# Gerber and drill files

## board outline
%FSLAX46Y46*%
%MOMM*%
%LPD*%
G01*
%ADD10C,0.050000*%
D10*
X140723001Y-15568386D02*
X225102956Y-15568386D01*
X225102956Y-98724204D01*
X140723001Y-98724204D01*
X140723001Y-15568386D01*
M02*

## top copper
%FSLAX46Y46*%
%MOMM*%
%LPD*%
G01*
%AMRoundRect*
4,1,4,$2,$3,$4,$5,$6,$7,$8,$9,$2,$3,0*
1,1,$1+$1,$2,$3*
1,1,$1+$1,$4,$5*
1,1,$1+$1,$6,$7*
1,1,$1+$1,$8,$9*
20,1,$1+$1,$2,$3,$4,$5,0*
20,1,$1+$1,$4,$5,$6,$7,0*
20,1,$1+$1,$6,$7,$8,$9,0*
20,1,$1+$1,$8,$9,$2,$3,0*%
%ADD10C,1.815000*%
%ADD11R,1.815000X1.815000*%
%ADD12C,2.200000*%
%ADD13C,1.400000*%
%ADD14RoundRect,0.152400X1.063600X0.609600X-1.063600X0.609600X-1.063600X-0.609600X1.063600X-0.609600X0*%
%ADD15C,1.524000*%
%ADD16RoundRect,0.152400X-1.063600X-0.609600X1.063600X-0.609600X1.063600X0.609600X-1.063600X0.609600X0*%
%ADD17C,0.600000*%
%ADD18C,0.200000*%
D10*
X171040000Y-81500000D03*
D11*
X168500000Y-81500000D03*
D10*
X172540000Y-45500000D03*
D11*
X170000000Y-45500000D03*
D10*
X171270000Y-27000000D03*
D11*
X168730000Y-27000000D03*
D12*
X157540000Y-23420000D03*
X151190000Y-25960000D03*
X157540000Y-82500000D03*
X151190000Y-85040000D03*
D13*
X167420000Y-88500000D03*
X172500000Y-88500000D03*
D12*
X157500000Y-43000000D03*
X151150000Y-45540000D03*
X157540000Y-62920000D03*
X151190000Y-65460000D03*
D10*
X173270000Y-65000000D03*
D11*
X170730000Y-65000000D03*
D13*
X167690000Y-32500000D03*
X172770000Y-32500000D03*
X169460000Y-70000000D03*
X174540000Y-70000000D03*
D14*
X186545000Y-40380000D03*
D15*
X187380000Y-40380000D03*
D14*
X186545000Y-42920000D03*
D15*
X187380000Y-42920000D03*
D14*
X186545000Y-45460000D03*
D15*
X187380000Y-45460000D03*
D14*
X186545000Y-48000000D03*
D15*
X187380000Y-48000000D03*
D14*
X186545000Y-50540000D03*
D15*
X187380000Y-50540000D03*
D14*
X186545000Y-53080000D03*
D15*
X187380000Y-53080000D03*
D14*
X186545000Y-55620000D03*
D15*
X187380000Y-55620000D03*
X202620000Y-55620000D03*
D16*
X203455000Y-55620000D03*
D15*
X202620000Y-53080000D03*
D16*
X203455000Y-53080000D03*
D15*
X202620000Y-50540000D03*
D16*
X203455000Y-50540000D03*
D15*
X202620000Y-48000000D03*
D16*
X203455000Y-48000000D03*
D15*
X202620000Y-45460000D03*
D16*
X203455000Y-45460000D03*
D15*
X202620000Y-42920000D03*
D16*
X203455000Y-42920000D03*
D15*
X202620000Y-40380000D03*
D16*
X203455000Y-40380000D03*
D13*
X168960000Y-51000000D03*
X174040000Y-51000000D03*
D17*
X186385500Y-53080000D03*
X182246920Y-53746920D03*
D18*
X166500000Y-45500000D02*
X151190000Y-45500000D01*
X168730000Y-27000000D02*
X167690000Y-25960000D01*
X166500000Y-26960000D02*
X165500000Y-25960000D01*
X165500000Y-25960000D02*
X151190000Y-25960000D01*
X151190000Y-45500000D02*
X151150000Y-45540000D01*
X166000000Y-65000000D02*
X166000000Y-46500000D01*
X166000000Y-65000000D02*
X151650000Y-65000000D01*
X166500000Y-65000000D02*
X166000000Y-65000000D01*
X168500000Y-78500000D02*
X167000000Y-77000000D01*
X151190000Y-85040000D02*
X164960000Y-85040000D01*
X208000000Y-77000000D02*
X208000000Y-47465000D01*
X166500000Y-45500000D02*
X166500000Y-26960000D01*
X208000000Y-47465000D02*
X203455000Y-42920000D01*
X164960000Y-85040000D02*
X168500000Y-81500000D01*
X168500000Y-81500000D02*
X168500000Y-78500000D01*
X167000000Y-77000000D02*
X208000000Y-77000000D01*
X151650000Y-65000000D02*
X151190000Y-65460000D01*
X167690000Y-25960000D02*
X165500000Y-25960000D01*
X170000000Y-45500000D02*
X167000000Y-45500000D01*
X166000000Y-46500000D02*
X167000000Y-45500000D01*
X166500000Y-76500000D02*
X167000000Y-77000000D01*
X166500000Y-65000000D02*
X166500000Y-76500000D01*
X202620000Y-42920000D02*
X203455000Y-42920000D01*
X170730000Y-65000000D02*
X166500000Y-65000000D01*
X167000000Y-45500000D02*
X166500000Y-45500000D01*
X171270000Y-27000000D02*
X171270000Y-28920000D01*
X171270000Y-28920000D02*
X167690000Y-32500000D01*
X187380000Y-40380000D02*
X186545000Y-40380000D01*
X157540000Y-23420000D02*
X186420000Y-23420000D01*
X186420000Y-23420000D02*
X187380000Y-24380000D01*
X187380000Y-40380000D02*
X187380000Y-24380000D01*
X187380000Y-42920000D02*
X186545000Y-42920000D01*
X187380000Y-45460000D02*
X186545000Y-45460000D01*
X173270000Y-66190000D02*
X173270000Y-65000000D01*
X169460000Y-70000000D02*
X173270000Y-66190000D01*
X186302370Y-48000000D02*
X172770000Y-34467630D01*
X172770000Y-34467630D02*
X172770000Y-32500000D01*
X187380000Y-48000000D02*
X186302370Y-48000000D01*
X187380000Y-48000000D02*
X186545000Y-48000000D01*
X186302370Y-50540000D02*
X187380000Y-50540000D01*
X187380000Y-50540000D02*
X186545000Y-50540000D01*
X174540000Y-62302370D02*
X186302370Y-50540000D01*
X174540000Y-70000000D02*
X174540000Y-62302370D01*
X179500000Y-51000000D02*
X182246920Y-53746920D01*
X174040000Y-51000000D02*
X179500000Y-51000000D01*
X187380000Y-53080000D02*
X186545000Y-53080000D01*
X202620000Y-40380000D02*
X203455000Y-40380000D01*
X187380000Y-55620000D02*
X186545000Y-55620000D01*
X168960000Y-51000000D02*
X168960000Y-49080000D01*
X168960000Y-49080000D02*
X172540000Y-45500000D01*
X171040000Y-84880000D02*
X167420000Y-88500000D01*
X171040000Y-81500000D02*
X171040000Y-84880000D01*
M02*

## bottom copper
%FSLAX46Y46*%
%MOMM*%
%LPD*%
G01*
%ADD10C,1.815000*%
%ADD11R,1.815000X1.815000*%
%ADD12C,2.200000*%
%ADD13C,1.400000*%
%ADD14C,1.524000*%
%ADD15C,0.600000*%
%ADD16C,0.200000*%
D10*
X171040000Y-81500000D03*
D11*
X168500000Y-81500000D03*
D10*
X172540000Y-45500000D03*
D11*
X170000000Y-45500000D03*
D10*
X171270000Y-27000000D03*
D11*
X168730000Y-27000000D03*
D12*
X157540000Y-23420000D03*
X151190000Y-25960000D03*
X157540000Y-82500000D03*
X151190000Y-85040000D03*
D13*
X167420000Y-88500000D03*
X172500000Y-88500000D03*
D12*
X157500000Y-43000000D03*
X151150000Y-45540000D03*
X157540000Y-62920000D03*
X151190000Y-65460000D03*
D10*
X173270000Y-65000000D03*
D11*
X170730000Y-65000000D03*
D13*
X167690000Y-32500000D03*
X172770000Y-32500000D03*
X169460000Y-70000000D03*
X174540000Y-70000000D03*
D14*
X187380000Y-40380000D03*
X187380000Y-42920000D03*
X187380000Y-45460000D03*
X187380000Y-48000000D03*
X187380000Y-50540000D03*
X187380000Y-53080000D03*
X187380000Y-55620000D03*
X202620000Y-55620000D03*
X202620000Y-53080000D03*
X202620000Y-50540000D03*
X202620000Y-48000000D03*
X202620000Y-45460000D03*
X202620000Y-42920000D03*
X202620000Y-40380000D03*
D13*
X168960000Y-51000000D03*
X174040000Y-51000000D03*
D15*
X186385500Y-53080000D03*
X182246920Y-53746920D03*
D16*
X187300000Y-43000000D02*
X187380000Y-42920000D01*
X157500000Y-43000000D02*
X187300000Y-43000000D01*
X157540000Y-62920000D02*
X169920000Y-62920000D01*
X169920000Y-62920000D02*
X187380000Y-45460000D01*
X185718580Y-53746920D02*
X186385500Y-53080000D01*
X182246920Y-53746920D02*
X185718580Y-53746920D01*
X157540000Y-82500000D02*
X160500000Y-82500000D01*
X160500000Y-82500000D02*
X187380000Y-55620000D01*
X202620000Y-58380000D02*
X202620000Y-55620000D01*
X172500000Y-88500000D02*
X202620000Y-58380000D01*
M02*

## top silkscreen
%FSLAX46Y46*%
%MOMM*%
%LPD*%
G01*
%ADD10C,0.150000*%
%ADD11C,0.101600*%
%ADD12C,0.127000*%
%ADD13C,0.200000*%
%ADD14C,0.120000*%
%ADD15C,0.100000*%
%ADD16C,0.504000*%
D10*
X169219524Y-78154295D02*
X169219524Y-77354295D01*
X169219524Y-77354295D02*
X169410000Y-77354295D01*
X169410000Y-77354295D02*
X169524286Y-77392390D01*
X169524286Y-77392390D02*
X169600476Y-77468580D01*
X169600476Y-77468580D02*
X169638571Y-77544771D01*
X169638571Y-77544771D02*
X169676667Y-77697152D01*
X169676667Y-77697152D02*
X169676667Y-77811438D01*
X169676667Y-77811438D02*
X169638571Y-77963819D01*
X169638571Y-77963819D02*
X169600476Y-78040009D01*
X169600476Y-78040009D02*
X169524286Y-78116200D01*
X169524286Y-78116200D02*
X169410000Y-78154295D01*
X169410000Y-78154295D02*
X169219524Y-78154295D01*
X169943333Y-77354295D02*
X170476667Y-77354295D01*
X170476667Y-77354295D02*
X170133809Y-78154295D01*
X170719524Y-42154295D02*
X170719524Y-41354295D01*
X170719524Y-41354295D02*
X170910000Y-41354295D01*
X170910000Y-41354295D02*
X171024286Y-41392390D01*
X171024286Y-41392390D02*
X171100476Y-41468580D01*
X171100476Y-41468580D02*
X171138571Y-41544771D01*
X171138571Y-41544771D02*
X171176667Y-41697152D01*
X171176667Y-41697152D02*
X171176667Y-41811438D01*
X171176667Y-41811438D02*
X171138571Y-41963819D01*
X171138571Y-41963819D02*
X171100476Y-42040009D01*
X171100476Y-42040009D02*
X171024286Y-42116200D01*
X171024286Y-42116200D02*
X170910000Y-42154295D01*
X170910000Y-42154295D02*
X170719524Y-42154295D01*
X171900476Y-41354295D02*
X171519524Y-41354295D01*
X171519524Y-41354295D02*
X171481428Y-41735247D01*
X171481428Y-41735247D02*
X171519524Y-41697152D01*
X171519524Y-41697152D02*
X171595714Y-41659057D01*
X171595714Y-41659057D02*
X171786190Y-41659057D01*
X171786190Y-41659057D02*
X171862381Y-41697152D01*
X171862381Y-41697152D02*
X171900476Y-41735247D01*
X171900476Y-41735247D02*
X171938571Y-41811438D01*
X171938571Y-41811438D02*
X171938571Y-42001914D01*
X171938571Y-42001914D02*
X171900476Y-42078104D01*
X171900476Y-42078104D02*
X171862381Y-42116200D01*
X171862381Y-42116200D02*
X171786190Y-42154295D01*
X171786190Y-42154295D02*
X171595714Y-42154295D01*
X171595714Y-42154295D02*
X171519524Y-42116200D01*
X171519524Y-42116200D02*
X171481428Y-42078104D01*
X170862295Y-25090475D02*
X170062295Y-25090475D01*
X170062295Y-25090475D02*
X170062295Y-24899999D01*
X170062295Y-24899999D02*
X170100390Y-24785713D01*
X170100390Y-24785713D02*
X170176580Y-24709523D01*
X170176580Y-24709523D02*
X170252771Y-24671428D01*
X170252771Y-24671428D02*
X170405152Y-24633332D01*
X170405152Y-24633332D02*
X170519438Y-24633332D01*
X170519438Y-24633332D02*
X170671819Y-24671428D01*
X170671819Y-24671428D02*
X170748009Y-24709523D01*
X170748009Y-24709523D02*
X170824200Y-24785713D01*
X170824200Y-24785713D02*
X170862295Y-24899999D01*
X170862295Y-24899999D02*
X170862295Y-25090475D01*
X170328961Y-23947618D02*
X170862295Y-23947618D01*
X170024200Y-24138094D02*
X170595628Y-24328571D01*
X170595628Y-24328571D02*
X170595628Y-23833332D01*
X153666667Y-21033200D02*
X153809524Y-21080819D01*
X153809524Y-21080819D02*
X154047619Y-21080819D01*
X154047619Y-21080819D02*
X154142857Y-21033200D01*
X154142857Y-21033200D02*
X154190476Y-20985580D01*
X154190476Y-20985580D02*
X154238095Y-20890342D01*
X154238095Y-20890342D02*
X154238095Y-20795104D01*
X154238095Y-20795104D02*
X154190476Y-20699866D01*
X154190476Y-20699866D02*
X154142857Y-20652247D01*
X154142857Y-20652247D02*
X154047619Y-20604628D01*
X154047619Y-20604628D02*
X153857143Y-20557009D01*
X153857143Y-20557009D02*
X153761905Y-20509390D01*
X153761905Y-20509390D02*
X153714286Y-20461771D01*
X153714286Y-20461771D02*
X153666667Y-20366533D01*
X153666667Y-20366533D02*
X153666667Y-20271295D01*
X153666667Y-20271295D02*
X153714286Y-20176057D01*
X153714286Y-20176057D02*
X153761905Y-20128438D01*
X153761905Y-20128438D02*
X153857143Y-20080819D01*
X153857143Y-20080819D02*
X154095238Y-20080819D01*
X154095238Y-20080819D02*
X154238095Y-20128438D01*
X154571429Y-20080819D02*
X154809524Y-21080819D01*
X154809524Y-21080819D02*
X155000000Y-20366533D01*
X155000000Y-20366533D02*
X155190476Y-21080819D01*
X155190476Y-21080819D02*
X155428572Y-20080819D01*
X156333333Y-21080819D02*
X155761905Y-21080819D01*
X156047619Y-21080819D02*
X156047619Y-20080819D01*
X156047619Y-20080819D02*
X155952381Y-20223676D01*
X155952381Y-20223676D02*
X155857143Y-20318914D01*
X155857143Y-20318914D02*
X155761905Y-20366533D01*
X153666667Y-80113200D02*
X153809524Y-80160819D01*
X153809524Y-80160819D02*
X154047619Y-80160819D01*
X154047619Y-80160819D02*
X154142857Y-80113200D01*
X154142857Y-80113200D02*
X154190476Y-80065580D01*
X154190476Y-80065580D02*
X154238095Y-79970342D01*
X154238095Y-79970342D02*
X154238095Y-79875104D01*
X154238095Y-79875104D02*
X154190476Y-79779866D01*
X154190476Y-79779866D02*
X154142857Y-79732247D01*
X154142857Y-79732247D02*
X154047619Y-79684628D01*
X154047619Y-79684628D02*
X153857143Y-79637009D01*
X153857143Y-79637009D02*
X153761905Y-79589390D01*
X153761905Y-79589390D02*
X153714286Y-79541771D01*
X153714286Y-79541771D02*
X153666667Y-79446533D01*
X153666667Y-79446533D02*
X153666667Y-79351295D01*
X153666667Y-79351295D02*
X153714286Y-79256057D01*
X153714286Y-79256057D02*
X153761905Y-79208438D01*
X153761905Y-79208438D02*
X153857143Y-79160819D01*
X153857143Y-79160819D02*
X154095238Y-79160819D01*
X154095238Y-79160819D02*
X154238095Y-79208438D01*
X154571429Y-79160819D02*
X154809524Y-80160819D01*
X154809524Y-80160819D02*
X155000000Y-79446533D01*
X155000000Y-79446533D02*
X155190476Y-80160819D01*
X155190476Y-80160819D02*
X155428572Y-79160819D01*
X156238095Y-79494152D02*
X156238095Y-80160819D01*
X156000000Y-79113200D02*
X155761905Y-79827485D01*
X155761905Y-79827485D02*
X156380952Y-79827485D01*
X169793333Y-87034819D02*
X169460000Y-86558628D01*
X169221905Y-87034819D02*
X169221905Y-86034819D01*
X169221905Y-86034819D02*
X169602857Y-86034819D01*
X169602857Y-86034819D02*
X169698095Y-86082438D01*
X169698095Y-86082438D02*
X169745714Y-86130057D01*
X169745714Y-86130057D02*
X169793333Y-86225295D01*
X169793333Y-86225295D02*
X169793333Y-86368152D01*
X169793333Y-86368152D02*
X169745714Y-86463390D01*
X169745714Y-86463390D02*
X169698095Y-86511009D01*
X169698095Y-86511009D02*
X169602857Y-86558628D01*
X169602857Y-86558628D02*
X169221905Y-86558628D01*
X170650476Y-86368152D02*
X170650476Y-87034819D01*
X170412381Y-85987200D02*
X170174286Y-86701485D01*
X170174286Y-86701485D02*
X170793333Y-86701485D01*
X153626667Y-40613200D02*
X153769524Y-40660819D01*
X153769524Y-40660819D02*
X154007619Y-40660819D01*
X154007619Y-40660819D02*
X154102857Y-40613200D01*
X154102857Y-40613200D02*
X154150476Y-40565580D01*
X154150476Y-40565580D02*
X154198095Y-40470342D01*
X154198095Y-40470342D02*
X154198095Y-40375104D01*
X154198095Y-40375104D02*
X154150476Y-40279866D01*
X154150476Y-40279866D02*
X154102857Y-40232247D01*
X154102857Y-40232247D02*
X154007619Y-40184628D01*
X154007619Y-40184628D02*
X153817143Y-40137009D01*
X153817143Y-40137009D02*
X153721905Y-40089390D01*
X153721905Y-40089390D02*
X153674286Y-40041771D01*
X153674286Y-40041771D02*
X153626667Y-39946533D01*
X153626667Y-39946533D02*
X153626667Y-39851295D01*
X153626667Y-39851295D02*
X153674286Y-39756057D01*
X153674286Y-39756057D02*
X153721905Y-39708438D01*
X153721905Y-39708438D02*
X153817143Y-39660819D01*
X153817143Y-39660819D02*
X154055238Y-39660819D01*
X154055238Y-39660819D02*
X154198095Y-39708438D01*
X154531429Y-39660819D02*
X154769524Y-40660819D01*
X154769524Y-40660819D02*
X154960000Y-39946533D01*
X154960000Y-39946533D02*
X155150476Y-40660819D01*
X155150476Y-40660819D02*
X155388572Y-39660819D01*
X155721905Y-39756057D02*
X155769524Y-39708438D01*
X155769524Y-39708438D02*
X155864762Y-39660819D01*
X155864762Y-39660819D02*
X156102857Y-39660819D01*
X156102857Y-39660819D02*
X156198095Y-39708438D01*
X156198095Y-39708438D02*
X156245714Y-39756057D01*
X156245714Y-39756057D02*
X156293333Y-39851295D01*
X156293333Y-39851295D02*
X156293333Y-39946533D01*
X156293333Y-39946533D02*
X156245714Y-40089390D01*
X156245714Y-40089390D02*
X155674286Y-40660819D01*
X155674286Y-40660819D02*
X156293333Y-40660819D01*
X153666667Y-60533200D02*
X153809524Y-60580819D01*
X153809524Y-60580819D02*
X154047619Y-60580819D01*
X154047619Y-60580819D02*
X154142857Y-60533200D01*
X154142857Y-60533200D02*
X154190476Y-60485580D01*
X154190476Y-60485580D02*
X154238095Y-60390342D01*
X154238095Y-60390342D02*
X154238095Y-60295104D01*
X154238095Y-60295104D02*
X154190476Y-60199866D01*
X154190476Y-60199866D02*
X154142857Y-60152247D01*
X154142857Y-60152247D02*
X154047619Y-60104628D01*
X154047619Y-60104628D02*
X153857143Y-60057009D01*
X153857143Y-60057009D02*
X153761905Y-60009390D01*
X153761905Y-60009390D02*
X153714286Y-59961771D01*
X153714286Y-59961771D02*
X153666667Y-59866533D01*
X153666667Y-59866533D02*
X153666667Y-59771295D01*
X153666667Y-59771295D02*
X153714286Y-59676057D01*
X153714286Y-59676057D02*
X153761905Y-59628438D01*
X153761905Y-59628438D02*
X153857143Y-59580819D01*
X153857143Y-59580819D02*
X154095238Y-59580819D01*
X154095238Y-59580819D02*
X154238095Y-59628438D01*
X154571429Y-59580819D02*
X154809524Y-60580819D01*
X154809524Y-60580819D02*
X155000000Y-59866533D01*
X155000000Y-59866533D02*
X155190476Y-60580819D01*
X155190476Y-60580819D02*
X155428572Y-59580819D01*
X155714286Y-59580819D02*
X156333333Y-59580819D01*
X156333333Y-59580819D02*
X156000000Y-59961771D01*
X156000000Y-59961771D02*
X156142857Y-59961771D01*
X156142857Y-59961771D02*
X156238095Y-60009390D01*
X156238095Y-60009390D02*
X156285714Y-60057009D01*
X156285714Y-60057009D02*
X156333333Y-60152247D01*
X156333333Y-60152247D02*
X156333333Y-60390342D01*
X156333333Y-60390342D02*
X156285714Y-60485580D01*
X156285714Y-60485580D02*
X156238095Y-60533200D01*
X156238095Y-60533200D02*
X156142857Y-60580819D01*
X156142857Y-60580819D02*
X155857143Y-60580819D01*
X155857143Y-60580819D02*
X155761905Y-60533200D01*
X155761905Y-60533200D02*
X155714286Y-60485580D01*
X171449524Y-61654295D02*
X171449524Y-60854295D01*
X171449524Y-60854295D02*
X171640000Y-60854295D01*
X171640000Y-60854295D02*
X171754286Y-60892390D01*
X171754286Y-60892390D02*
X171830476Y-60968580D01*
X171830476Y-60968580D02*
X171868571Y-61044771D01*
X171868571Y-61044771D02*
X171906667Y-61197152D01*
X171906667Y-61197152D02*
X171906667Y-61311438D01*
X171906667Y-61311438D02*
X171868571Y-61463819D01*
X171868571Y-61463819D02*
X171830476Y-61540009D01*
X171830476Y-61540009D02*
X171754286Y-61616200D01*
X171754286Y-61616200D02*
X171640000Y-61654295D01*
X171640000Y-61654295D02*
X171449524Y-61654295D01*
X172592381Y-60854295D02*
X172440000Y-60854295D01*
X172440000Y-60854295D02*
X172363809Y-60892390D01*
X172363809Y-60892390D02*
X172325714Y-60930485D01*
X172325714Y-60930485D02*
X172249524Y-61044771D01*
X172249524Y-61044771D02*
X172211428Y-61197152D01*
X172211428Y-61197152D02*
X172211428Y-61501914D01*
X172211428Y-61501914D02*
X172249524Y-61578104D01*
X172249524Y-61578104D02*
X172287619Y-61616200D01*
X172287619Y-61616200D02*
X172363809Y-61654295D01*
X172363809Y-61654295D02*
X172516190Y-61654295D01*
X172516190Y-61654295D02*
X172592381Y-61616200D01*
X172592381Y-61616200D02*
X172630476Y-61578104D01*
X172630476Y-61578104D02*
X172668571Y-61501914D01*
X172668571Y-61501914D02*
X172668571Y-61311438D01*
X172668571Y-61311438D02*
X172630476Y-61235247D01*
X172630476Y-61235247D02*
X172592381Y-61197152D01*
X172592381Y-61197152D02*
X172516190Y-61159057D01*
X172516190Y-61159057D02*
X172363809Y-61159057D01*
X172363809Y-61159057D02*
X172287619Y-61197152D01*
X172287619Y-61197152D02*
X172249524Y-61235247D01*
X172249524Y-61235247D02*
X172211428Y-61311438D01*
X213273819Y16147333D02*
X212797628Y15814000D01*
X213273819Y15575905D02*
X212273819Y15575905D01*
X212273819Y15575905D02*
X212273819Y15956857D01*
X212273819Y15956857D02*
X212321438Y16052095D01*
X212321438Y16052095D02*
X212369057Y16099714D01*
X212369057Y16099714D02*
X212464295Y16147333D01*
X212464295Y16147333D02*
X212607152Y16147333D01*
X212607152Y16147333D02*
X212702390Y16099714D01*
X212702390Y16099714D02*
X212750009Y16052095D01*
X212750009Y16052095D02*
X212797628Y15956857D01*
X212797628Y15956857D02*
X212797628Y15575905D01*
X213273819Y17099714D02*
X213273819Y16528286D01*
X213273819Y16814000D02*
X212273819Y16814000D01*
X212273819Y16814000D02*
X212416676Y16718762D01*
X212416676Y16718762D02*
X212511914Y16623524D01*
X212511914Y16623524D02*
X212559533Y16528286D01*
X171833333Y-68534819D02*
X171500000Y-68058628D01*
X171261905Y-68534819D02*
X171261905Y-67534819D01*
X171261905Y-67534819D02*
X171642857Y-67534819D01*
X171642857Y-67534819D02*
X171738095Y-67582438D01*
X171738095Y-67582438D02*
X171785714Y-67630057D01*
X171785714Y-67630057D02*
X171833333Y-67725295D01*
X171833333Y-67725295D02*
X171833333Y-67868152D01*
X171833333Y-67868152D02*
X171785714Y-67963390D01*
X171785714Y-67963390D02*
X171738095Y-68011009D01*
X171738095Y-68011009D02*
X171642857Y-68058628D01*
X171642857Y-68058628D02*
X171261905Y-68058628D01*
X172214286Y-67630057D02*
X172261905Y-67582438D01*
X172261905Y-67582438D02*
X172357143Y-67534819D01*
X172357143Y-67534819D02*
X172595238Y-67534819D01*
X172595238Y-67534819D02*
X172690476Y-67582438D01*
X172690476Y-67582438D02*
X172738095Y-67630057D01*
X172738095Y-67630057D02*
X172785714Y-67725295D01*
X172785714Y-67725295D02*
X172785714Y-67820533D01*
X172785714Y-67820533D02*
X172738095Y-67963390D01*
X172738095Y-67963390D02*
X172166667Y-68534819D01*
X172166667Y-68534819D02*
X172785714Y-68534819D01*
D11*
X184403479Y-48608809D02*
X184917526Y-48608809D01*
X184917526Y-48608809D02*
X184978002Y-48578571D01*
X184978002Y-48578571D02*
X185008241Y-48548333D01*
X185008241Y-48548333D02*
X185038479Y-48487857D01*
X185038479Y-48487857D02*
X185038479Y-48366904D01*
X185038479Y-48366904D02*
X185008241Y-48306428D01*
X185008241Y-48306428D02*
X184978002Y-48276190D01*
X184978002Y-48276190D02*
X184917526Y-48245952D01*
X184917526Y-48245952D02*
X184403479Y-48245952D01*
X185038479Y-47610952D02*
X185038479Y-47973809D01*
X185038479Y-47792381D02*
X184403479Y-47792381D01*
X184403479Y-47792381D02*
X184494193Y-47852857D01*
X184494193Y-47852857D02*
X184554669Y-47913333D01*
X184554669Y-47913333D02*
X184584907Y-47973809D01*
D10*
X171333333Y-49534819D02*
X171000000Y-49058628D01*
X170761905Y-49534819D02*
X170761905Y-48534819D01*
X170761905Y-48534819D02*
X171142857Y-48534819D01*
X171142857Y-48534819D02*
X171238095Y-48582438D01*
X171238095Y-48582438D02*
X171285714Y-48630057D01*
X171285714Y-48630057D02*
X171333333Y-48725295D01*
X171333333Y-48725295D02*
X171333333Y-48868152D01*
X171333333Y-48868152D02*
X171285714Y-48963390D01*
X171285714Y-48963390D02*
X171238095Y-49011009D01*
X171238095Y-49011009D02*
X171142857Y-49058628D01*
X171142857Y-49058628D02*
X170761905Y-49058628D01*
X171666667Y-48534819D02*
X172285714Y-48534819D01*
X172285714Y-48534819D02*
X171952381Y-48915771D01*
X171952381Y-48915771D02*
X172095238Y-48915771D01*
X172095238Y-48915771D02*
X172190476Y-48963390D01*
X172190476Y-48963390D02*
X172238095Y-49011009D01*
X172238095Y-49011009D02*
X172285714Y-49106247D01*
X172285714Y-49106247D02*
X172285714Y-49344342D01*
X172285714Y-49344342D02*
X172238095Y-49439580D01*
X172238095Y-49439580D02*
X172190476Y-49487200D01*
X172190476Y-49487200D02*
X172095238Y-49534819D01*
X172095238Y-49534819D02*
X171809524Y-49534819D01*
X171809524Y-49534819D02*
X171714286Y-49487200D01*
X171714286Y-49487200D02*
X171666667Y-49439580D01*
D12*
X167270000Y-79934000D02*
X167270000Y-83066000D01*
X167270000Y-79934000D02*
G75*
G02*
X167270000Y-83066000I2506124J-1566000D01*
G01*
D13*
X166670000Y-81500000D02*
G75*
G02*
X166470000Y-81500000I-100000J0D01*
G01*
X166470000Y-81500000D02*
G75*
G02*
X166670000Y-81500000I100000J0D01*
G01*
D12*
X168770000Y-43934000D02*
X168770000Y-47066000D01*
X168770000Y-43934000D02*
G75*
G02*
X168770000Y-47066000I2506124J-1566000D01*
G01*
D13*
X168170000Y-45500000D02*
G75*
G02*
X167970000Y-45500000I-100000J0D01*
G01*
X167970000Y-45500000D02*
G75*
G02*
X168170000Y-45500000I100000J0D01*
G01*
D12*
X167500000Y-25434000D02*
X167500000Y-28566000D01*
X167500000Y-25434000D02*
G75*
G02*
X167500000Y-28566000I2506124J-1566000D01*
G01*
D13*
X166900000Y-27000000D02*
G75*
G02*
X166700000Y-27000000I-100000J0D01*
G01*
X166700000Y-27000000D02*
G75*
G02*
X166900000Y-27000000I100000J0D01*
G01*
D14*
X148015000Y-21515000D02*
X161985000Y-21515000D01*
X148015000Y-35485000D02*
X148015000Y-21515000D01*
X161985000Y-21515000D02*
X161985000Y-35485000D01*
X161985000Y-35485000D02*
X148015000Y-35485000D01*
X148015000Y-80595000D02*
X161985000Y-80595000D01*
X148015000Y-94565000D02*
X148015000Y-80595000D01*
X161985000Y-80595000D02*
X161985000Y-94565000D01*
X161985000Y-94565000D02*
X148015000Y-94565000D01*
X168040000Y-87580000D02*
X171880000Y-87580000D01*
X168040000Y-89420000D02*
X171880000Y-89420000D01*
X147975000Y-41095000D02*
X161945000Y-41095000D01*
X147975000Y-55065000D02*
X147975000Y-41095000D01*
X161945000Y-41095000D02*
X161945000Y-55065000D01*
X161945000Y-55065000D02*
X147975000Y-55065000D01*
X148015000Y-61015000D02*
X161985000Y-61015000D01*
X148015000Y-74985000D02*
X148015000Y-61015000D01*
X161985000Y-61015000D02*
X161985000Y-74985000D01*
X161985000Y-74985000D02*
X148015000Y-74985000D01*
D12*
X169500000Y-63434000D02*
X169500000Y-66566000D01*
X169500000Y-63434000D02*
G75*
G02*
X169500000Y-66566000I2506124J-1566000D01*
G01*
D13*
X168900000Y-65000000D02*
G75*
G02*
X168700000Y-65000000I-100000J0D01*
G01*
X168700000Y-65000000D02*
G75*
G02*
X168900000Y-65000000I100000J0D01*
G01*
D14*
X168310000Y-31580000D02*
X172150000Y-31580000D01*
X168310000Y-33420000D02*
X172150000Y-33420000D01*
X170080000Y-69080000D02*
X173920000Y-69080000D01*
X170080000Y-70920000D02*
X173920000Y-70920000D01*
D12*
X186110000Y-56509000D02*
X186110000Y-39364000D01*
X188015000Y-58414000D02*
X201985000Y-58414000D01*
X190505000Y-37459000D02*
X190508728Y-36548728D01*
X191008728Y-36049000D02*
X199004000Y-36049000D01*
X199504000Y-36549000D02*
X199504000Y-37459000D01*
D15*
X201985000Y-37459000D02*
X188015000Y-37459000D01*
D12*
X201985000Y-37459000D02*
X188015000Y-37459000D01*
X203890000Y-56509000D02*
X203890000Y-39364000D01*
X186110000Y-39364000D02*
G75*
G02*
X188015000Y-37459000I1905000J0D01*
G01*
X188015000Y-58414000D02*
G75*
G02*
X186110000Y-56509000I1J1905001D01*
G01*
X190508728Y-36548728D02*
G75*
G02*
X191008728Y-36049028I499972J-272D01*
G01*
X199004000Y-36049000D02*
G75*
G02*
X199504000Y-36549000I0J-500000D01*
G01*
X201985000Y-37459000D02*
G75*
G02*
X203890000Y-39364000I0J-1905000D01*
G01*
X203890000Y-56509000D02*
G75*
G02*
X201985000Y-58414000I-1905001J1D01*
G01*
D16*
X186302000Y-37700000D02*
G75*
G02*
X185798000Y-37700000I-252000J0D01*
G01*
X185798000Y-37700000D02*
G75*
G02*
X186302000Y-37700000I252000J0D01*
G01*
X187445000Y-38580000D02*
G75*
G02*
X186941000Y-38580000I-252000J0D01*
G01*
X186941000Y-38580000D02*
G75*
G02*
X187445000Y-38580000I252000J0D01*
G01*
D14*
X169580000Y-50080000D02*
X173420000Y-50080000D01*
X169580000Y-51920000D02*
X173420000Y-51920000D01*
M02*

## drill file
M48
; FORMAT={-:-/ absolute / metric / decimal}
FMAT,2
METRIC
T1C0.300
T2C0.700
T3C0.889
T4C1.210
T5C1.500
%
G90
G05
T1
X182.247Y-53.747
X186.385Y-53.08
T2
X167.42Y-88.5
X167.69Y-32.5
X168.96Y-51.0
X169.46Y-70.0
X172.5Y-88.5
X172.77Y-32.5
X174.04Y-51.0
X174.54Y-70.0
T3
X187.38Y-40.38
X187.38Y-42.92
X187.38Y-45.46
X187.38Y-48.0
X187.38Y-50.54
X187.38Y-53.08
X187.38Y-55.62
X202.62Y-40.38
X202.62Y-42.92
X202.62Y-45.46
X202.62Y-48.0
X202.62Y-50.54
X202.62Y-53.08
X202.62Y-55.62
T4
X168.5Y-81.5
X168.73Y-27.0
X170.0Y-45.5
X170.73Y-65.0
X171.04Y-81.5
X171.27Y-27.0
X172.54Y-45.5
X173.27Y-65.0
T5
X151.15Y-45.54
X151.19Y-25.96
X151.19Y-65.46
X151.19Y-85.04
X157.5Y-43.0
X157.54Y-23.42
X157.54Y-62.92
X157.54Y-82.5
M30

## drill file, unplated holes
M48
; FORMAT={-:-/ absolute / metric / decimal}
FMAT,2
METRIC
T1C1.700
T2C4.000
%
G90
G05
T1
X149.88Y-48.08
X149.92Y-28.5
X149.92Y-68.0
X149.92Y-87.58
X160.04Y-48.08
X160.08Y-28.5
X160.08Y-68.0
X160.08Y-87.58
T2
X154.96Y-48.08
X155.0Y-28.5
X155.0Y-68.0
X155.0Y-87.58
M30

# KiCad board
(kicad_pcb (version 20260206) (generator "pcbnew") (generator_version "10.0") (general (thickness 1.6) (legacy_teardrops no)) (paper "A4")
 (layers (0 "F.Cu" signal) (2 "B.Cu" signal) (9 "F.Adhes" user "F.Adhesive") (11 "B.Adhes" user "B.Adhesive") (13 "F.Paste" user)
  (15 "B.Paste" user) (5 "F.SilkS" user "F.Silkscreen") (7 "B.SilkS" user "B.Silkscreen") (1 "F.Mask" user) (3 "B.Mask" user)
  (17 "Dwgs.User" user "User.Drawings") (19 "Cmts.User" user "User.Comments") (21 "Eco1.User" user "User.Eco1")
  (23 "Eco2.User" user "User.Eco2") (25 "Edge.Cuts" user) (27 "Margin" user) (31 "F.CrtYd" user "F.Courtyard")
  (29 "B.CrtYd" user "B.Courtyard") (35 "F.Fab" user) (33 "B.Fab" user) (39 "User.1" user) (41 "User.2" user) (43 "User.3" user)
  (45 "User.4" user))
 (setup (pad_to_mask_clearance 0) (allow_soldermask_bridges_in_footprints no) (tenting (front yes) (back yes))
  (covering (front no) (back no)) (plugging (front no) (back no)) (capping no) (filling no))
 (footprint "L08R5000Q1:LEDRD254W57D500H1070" (layer "F.Cu") (at 169.77 81.5)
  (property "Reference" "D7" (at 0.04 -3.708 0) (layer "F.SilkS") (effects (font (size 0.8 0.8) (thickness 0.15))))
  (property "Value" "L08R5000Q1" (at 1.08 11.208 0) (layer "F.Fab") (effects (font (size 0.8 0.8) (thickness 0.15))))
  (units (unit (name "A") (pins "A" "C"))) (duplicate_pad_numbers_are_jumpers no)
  (fp_line (start -2.5 -1.566) (end -2.5 1.566) (stroke (width 0.127) (type solid)) (layer "F.SilkS"))
  (fp_arc (start -2.5 -1.566) (mid 2.961291 0) (end -2.5 1.566) (stroke (width 0.127) (type solid)) (layer "F.SilkS"))
  (fp_circle (center -3.2 0) (end -3.1 0) (stroke (width 0.2) (type solid)) (fill no) (layer "F.SilkS"))
  (pad "A" thru_hole circle (at 1.27 0) (size 1.815 1.815) (drill 1.21) (layers "*.Cu" "*.Mask") (remove_unused_layers no)
   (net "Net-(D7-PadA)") (solder_mask_margin 0.102))
  (pad "C" thru_hole rect (at -1.27 0) (size 1.815 1.815) (drill 1.21) (layers "*.Cu" "*.Mask") (remove_unused_layers no) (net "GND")
   (solder_mask_margin 0.102)))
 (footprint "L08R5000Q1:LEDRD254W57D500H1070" (layer "F.Cu") (at 171.27 45.5)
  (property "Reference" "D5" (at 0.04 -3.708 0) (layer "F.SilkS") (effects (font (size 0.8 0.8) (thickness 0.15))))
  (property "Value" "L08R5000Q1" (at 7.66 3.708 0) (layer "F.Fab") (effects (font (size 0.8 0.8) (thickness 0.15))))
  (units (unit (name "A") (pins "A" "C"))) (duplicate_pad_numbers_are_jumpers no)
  (fp_line (start -2.5 -1.566) (end -2.5 1.566) (stroke (width 0.127) (type solid)) (layer "F.SilkS"))
  (fp_arc (start -2.5 -1.566) (mid 2.961291 0) (end -2.5 1.566) (stroke (width 0.127) (type solid)) (layer "F.SilkS"))
  (fp_circle (center -3.2 0) (end -3.1 0) (stroke (width 0.2) (type solid)) (fill no) (layer "F.SilkS"))
  (pad "A" thru_hole circle (at 1.27 0) (size 1.815 1.815) (drill 1.21) (layers "*.Cu" "*.Mask") (remove_unused_layers no)
   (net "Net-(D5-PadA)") (solder_mask_margin 0.102))
  (pad "C" thru_hole rect (at -1.27 0) (size 1.815 1.815) (drill 1.21) (layers "*.Cu" "*.Mask") (remove_unused_layers no) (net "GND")
   (solder_mask_margin 0.102)))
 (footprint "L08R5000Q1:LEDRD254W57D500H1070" (layer "F.Cu") (at 170 27)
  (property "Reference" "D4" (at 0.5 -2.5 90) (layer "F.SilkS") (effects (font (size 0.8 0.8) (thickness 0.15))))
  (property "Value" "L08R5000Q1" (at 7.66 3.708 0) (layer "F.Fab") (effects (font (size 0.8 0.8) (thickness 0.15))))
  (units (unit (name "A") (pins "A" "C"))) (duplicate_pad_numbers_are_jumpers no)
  (fp_line (start -2.5 -1.566) (end -2.5 1.566) (stroke (width 0.127) (type solid)) (layer "F.SilkS"))
  (fp_arc (start -2.5 -1.566) (mid 2.961291 0) (end -2.5 1.566) (stroke (width 0.127) (type solid)) (layer "F.SilkS"))
  (fp_circle (center -3.2 0) (end -3.1 0) (stroke (width 0.2) (type solid)) (fill no) (layer "F.SilkS"))
  (pad "A" thru_hole circle (at 1.27 0) (size 1.815 1.815) (drill 1.21) (layers "*.Cu" "*.Mask") (remove_unused_layers no)
   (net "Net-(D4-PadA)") (solder_mask_margin 0.102))
  (pad "C" thru_hole rect (at -1.27 0) (size 1.815 1.815) (drill 1.21) (layers "*.Cu" "*.Mask") (remove_unused_layers no) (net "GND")
   (solder_mask_margin 0.102)))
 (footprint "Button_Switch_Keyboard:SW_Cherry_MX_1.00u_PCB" (layer "F.Cu") (at 157.54 23.42)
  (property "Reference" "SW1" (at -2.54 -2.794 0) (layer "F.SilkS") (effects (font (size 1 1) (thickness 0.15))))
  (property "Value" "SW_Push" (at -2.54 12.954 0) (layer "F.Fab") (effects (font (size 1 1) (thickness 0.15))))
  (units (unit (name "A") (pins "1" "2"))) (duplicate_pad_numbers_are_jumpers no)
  (fp_line (start -9.525 -1.905) (end 4.445 -1.905) (stroke (width 0.12) (type solid)) (layer "F.SilkS"))
  (fp_line (start -9.525 12.065) (end -9.525 -1.905) (stroke (width 0.12) (type solid)) (layer "F.SilkS"))
  (fp_line (start 4.445 -1.905) (end 4.445 12.065) (stroke (width 0.12) (type solid)) (layer "F.SilkS"))
  (fp_line (start 4.445 12.065) (end -9.525 12.065) (stroke (width 0.12) (type solid)) (layer "F.SilkS"))
  (pad "" np_thru_hole circle (at -7.62 5.08) (size 1.7 1.7) (drill 1.7) (layers "*.Cu" "*.Mask"))
  (pad "" np_thru_hole circle (at -2.54 5.08) (size 4 4) (drill 4) (layers "*.Cu" "*.Mask"))
  (pad "" np_thru_hole circle (at 2.54 5.08) (size 1.7 1.7) (drill 1.7) (layers "*.Cu" "*.Mask"))
  (pad "1" thru_hole circle (at 0 0) (size 2.2 2.2) (drill 1.5) (layers "*.Cu" "*.Mask") (remove_unused_layers no) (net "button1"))
  (pad "2" thru_hole circle (at -6.35 2.54) (size 2.2 2.2) (drill 1.5) (layers "*.Cu" "*.Mask") (remove_unused_layers no) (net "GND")))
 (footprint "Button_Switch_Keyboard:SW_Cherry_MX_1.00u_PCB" (layer "F.Cu") (at 157.54 82.5)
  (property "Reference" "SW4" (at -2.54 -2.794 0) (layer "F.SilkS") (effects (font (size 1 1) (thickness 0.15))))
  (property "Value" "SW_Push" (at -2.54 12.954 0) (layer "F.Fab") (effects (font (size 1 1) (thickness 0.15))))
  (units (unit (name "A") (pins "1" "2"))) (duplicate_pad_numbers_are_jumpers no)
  (fp_line (start -9.525 -1.905) (end 4.445 -1.905) (stroke (width 0.12) (type solid)) (layer "F.SilkS"))
  (fp_line (start -9.525 12.065) (end -9.525 -1.905) (stroke (width 0.12) (type solid)) (layer "F.SilkS"))
  (fp_line (start 4.445 -1.905) (end 4.445 12.065) (stroke (width 0.12) (type solid)) (layer "F.SilkS"))
  (fp_line (start 4.445 12.065) (end -9.525 12.065) (stroke (width 0.12) (type solid)) (layer "F.SilkS"))
  (pad "" np_thru_hole circle (at -7.62 5.08) (size 1.7 1.7) (drill 1.7) (layers "*.Cu" "*.Mask"))
  (pad "" np_thru_hole circle (at -2.54 5.08) (size 4 4) (drill 4) (layers "*.Cu" "*.Mask"))
  (pad "" np_thru_hole circle (at 2.54 5.08) (size 1.7 1.7) (drill 1.7) (layers "*.Cu" "*.Mask"))
  (pad "1" thru_hole circle (at 0 0) (size 2.2 2.2) (drill 1.5) (layers "*.Cu" "*.Mask") (remove_unused_layers no) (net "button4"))
  (pad "2" thru_hole circle (at -6.35 2.54) (size 2.2 2.2) (drill 1.5) (layers "*.Cu" "*.Mask") (remove_unused_layers no) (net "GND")))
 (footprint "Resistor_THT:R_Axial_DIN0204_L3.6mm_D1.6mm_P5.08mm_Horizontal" (layer "F.Cu") (at 167.42 88.5)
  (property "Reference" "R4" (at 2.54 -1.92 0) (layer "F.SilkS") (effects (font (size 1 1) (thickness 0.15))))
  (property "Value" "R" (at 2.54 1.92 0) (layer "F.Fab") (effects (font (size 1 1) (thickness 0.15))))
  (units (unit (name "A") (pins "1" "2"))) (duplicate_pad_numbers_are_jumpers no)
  (fp_line (start 0.62 -0.92) (end 4.46 -0.92) (stroke (width 0.12) (type solid)) (layer "F.SilkS"))
  (fp_line (start 0.62 0.92) (end 4.46 0.92) (stroke (width 0.12) (type solid)) (layer "F.SilkS"))
  (pad "1" thru_hole circle (at 0 0) (size 1.4 1.4) (drill 0.7) (layers "*.Cu" "*.Mask") (remove_unused_layers no) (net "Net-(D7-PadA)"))
  (pad "2" thru_hole circle (at 5.08 0) (size 1.4 1.4) (drill 0.7) (layers "*.Cu" "*.Mask") (remove_unused_layers no) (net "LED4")))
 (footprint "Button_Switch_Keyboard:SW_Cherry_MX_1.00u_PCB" (layer "F.Cu") (at 157.5 43)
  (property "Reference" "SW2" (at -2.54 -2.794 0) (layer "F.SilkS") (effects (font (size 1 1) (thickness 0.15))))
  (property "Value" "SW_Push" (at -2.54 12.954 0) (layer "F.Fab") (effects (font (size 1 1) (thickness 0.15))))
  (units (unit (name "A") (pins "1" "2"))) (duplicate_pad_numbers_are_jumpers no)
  (fp_line (start -9.525 -1.905) (end 4.445 -1.905) (stroke (width 0.12) (type solid)) (layer "F.SilkS"))
  (fp_line (start -9.525 12.065) (end -9.525 -1.905) (stroke (width 0.12) (type solid)) (layer "F.SilkS"))
  (fp_line (start 4.445 -1.905) (end 4.445 12.065) (stroke (width 0.12) (type solid)) (layer "F.SilkS"))
  (fp_line (start 4.445 12.065) (end -9.525 12.065) (stroke (width 0.12) (type solid)) (layer "F.SilkS"))
  (pad "" np_thru_hole circle (at -7.62 5.08) (size 1.7 1.7) (drill 1.7) (layers "*.Cu" "*.Mask"))
  (pad "" np_thru_hole circle (at -2.54 5.08) (size 4 4) (drill 4) (layers "*.Cu" "*.Mask"))
  (pad "" np_thru_hole circle (at 2.54 5.08) (size 1.7 1.7) (drill 1.7) (layers "*.Cu" "*.Mask"))
  (pad "1" thru_hole circle (at 0 0) (size 2.2 2.2) (drill 1.5) (layers "*.Cu" "*.Mask") (remove_unused_layers no) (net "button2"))
  (pad "2" thru_hole circle (at -6.35 2.54) (size 2.2 2.2) (drill 1.5) (layers "*.Cu" "*.Mask") (remove_unused_layers no) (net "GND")))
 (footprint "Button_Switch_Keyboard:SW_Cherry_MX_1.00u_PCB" (layer "F.Cu") (at 157.54 62.92)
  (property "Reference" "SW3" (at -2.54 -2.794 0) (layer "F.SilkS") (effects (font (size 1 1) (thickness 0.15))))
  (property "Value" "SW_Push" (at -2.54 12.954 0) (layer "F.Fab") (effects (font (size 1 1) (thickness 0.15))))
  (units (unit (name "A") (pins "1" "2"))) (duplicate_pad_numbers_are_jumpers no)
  (fp_line (start -9.525 -1.905) (end 4.445 -1.905) (stroke (width 0.12) (type solid)) (layer "F.SilkS"))
  (fp_line (start -9.525 12.065) (end -9.525 -1.905) (stroke (width 0.12) (type solid)) (layer "F.SilkS"))
  (fp_line (start 4.445 -1.905) (end 4.445 12.065) (stroke (width 0.12) (type solid)) (layer "F.SilkS"))
  (fp_line (start 4.445 12.065) (end -9.525 12.065) (stroke (width 0.12) (type solid)) (layer "F.SilkS"))
  (pad "" np_thru_hole circle (at -7.62 5.08) (size 1.7 1.7) (drill 1.7) (layers "*.Cu" "*.Mask"))
  (pad "" np_thru_hole circle (at -2.54 5.08) (size 4 4) (drill 4) (layers "*.Cu" "*.Mask"))
  (pad "" np_thru_hole circle (at 2.54 5.08) (size 1.7 1.7) (drill 1.7) (layers "*.Cu" "*.Mask"))
  (pad "1" thru_hole circle (at 0 0) (size 2.2 2.2) (drill 1.5) (layers "*.Cu" "*.Mask") (remove_unused_layers no) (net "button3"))
  (pad "2" thru_hole circle (at -6.35 2.54) (size 2.2 2.2) (drill 1.5) (layers "*.Cu" "*.Mask") (remove_unused_layers no) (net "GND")))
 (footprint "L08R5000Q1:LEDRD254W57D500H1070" (layer "F.Cu") (at 172 65)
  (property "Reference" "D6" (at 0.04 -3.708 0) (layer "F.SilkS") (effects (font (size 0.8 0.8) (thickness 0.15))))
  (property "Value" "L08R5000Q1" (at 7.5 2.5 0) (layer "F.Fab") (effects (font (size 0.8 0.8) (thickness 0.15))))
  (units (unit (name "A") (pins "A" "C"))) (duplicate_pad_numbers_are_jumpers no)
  (fp_line (start -2.5 -1.566) (end -2.5 1.566) (stroke (width 0.127) (type solid)) (layer "F.SilkS"))
  (fp_arc (start -2.5 -1.566) (mid 2.961291 0) (end -2.5 1.566) (stroke (width 0.127) (type solid)) (layer "F.SilkS"))
  (fp_circle (center -3.2 0) (end -3.1 0) (stroke (width 0.2) (type solid)) (fill no) (layer "F.SilkS"))
  (pad "A" thru_hole circle (at 1.27 0) (size 1.815 1.815) (drill 1.21) (layers "*.Cu" "*.Mask") (remove_unused_layers no)
   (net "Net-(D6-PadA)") (solder_mask_margin 0.102))
  (pad "C" thru_hole rect (at -1.27 0) (size 1.815 1.815) (drill 1.21) (layers "*.Cu" "*.Mask") (remove_unused_layers no) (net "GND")
   (solder_mask_margin 0.102)))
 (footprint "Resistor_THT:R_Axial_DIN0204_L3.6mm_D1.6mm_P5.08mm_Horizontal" (layer "F.Cu") (at 167.69 32.5)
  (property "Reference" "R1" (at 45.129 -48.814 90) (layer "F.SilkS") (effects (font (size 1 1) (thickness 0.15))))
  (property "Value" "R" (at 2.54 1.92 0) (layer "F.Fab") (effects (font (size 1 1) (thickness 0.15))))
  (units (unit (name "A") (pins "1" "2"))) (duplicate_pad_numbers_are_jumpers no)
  (fp_line (start 0.62 -0.92) (end 4.46 -0.92) (stroke (width 0.12) (type solid)) (layer "F.SilkS"))
  (fp_line (start 0.62 0.92) (end 4.46 0.92) (stroke (width 0.12) (type solid)) (layer "F.SilkS"))
  (pad "1" thru_hole circle (at 0 0) (size 1.4 1.4) (drill 0.7) (layers "*.Cu" "*.Mask") (remove_unused_layers no) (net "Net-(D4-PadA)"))
  (pad "2" thru_hole circle (at 5.08 0) (size 1.4 1.4) (drill 0.7) (layers "*.Cu" "*.Mask") (remove_unused_layers no) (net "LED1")))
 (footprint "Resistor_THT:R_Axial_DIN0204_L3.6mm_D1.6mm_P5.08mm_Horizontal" (layer "F.Cu") (at 169.46 70)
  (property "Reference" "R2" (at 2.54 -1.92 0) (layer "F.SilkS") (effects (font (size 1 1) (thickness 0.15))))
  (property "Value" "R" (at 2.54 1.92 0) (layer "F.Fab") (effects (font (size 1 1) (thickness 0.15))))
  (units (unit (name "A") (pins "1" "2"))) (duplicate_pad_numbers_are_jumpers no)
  (fp_line (start 0.62 -0.92) (end 4.46 -0.92) (stroke (width 0.12) (type solid)) (layer "F.SilkS"))
  (fp_line (start 0.62 0.92) (end 4.46 0.92) (stroke (width 0.12) (type solid)) (layer "F.SilkS"))
  (pad "1" thru_hole circle (at 0 0) (size 1.4 1.4) (drill 0.7) (layers "*.Cu" "*.Mask") (remove_unused_layers no) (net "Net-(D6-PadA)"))
  (pad "2" thru_hole circle (at 5.08 0) (size 1.4 1.4) (drill 0.7) (layers "*.Cu" "*.Mask") (remove_unused_layers no) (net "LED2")))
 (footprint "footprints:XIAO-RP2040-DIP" (layer "F.Cu") (at 195 48 90)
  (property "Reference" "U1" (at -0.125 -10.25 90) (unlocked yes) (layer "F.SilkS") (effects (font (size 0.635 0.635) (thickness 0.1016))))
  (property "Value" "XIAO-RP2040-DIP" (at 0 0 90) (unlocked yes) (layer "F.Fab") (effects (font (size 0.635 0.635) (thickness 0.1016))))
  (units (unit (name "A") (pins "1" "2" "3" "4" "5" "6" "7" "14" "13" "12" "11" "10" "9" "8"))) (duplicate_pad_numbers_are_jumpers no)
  (fp_line (start -8.509 -8.89) (end 8.636 -8.89) (stroke (width 0.127) (type solid)) (layer "F.SilkS"))
  (fp_line (start -10.414 -6.985) (end -10.414 6.985) (stroke (width 0.127) (type solid)) (layer "F.SilkS"))
  (fp_line (start 10.541 -4.495) (end 11.451272 -4.491272) (stroke (width 0.127) (type solid)) (layer "F.SilkS"))
  (fp_line (start 11.951 -3.991272) (end 11.951 4.004) (stroke (width 0.127) (type solid)) (layer "F.SilkS"))
  (fp_line (start 11.451 4.504) (end 10.541 4.504) (stroke (width 0.127) (type solid)) (layer "F.SilkS"))
  (fp_line (start 10.541 6.985) (end 10.541 -6.985) (stroke (width 0.1) (type solid)) (layer "F.SilkS"))
  (fp_line (start 10.541 6.985) (end 10.541 -6.985) (stroke (width 0.127) (type solid)) (layer "F.SilkS"))
  (fp_line (start -8.509 8.89) (end 8.636 8.89) (stroke (width 0.127) (type solid)) (layer "F.SilkS"))
  (fp_arc (start 8.636 -8.89) (mid 9.983038 -8.332038) (end 10.541 -6.985) (stroke (width 0.127) (type solid)) (layer "F.SilkS"))
  (fp_arc (start -10.414 -6.985) (mid -9.856038 -8.332038) (end -8.509 -8.89) (stroke (width 0.127) (type solid)) (layer "F.SilkS"))
  (fp_arc (start 11.451272 -4.491272) (mid 11.804644 -4.344724) (end 11.951 -3.991272) (stroke (width 0.127) (type default))
   (layer "F.SilkS"))
  (fp_arc (start 11.951 4.004) (mid 11.804553 4.357553) (end 11.451 4.504) (stroke (width 0.127) (type default)) (layer "F.SilkS"))
  (fp_arc (start 10.541 6.985) (mid 9.983038 8.332038) (end 8.636 8.89) (stroke (width 0.127) (type solid)) (layer "F.SilkS"))
  (fp_arc (start -8.509 8.89) (mid -9.856038 8.332038) (end -10.414 6.985) (stroke (width 0.127) (type solid)) (layer "F.SilkS"))
  (fp_circle (center 10.3 -8.95) (end 10.554 -8.95) (stroke (width 0.5) (type solid)) (fill yes) (layer "F.SilkS"))
  (fp_circle (center 9.42 -7.807) (end 9.674 -7.807) (stroke (width 0.5) (type solid)) (fill yes) (layer "F.SilkS"))
  (pad "1" smd roundrect (at 7.62 -8.455 180) (size 2.432 1.524) (layers "F.Cu" "F.Mask") (roundrect_rratio 0.1) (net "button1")
   (thermal_bridge_angle 45))
  (pad "1" thru_hole circle (at 7.62 -7.62 180) (size 1.524 1.524) (drill 0.889) (layers "*.Cu" "*.Mask") (remove_unused_layers no)
   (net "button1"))
  (pad "2" smd roundrect (at 5.08 -8.455 180) (size 2.432 1.524) (layers "F.Cu" "F.Mask") (roundrect_rratio 0.1) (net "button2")
   (thermal_bridge_angle 45))
  (pad "2" thru_hole circle (at 5.08 -7.62 180) (size 1.524 1.524) (drill 0.889) (layers "*.Cu" "*.Mask") (remove_unused_layers no)
   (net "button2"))
  (pad "3" smd roundrect (at 2.54 -8.455 180) (size 2.432 1.524) (layers "F.Cu" "F.Mask") (roundrect_rratio 0.1) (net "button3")
   (thermal_bridge_angle 45))
  (pad "3" thru_hole circle (at 2.54 -7.62 180) (size 1.524 1.524) (drill 0.889) (layers "*.Cu" "*.Mask") (remove_unused_layers no)
   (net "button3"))
  (pad "4" smd roundrect (at 0 -8.455 180) (size 2.432 1.524) (layers "F.Cu" "F.Mask") (roundrect_rratio 0.1) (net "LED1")
   (thermal_bridge_angle 45))
  (pad "4" thru_hole circle (at 0 -7.62 180) (size 1.524 1.524) (drill 0.889) (layers "*.Cu" "*.Mask") (remove_unused_layers no)
   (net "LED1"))
  (pad "5" smd roundrect (at -2.54 -8.455 180) (size 2.432 1.524) (layers "F.Cu" "F.Mask") (roundrect_rratio 0.1) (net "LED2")
   (thermal_bridge_angle 45))
  (pad "5" thru_hole circle (at -2.54 -7.62 180) (size 1.524 1.524) (drill 0.889) (layers "*.Cu" "*.Mask") (remove_unused_layers no)
   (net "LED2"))
  (pad "6" smd roundrect (at -5.08 -8.455 180) (size 2.432 1.524) (layers "F.Cu" "F.Mask") (roundrect_rratio 0.1) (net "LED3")
   (thermal_bridge_angle 45))
  (pad "6" thru_hole circle (at -5.08 -7.62 180) (size 1.524 1.524) (drill 0.889) (layers "*.Cu" "*.Mask") (remove_unused_layers no)
   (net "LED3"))
  (pad "7" smd roundrect (at -7.62 -8.455 180) (size 2.432 1.524) (layers "F.Cu" "F.Mask") (roundrect_rratio 0.1) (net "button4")
   (thermal_bridge_angle 45))
  (pad "7" thru_hole circle (at -7.62 -7.62 180) (size 1.524 1.524) (drill 0.889) (layers "*.Cu" "*.Mask") (remove_unused_layers no)
   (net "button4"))
  (pad "8" thru_hole circle (at -7.62 7.62) (size 1.524 1.524) (drill 0.889) (layers "*.Cu" "*.Mask") (remove_unused_layers no) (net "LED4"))
  (pad "8" smd roundrect (at -7.62 8.455) (size 2.432 1.524) (layers "F.Cu" "F.Mask") (roundrect_rratio 0.1) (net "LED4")
   (thermal_bridge_angle 45))
  (pad "9" thru_hole circle (at -5.08 7.62) (size 1.524 1.524) (drill 0.889) (layers "*.Cu" "*.Mask") (remove_unused_layers no)
   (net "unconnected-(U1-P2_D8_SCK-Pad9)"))
  (pad "9" smd roundrect (at -5.08 8.455) (size 2.432 1.524) (layers "F.Cu" "F.Mask") (roundrect_rratio 0.1)
   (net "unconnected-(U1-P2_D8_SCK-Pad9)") (thermal_bridge_angle 45))
  (pad "10" thru_hole circle (at -2.54 7.62) (size 1.524 1.524) (drill 0.889) (layers "*.Cu" "*.Mask") (remove_unused_layers no)
   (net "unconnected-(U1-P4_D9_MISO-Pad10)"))
  (pad "10" smd roundrect (at -2.54 8.455) (size 2.432 1.524) (layers "F.Cu" "F.Mask") (roundrect_rratio 0.1)
   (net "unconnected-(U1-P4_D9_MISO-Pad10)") (thermal_bridge_angle 45))
  (pad "11" thru_hole circle (at 0 7.62) (size 1.524 1.524) (drill 0.889) (layers "*.Cu" "*.Mask") (remove_unused_layers no)
   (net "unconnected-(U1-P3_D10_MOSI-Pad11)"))
  (pad "11" smd roundrect (at 0 8.455) (size 2.432 1.524) (layers "F.Cu" "F.Mask") (roundrect_rratio 0.1)
   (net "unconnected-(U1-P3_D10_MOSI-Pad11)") (thermal_bridge_angle 45))
  (pad "12" thru_hole circle (at 2.54 7.62) (size 1.524 1.524) (drill 0.889) (layers "*.Cu" "*.Mask") (remove_unused_layers no)
   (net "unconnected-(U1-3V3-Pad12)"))
  (pad "12" smd roundrect (at 2.54 8.455) (size 2.432 1.524) (layers "F.Cu" "F.Mask") (roundrect_rratio 0.1)
   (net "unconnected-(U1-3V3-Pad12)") (thermal_bridge_angle 45))
  (pad "13" thru_hole circle (at 5.08 7.62) (size 1.524 1.524) (drill 0.889) (layers "*.Cu" "*.Mask") (remove_unused_layers no) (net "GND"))
  (pad "13" smd roundrect (at 5.08 8.455) (size 2.432 1.524) (layers "F.Cu" "F.Mask") (roundrect_rratio 0.1) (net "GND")
   (thermal_bridge_angle 45))
  (pad "14" thru_hole circle (at 7.62 7.62) (size 1.524 1.524) (drill 0.889) (layers "*.Cu" "*.Mask") (remove_unused_layers no)
   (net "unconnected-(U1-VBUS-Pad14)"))
  (pad "14" smd roundrect (at 7.62 8.455) (size 2.432 1.524) (layers "F.Cu" "F.Mask") (roundrect_rratio 0.1)
   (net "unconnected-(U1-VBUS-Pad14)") (thermal_bridge_angle 45)))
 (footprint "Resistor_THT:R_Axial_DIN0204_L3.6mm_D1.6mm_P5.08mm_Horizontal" (layer "F.Cu") (at 168.96 51)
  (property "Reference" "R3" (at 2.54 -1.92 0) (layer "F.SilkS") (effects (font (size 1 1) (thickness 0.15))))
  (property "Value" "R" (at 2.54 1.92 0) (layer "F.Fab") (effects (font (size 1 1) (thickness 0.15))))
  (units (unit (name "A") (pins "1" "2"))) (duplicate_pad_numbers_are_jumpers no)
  (fp_line (start 0.62 -0.92) (end 4.46 -0.92) (stroke (width 0.12) (type solid)) (layer "F.SilkS"))
  (fp_line (start 0.62 0.92) (end 4.46 0.92) (stroke (width 0.12) (type solid)) (layer "F.SilkS"))
  (pad "1" thru_hole circle (at 0 0) (size 1.4 1.4) (drill 0.7) (layers "*.Cu" "*.Mask") (remove_unused_layers no) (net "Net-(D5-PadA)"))
  (pad "2" thru_hole circle (at 5.08 0) (size 1.4 1.4) (drill 0.7) (layers "*.Cu" "*.Mask") (remove_unused_layers no) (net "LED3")))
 (gr_rect (start 140.723001 15.568386) (end 225.102956 98.724204) (stroke (width 0.05) (type default)) (fill no) (layer "Edge.Cuts"))
 (segment (start 166.5 45.5) (end 151.19 45.5) (width 0.2) (layer "F.Cu") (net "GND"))
 (segment (start 168.73 27) (end 167.69 25.96) (width 0.2) (layer "F.Cu") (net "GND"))
 (segment (start 166.5 26.96) (end 165.5 25.96) (width 0.2) (layer "F.Cu") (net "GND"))
 (segment (start 165.5 25.96) (end 151.19 25.96) (width 0.2) (layer "F.Cu") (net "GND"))
 (segment (start 151.19 45.5) (end 151.15 45.54) (width 0.2) (layer "F.Cu") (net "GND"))
 (segment (start 166 65) (end 166 46.5) (width 0.2) (layer "F.Cu") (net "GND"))
 (segment (start 166 65) (end 151.65 65) (width 0.2) (layer "F.Cu") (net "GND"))
 (segment (start 166.5 65) (end 166 65) (width 0.2) (layer "F.Cu") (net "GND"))
 (segment (start 168.5 78.5) (end 167 77) (width 0.2) (layer "F.Cu") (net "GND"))
 (segment (start 151.19 85.04) (end 164.96 85.04) (width 0.2) (layer "F.Cu") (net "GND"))
 (segment (start 208 77) (end 208 47.465) (width 0.2) (layer "F.Cu") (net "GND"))
 (segment (start 166.5 45.5) (end 166.5 26.96) (width 0.2) (layer "F.Cu") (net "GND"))
 (segment (start 208 47.465) (end 203.455 42.92) (width 0.2) (layer "F.Cu") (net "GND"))
 (segment (start 164.96 85.04) (end 168.5 81.5) (width 0.2) (layer "F.Cu") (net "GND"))
 (segment (start 168.5 81.5) (end 168.5 78.5) (width 0.2) (layer "F.Cu") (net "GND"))
 (segment (start 167 77) (end 208 77) (width 0.2) (layer "F.Cu") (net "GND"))
 (segment (start 151.65 65) (end 151.19 65.46) (width 0.2) (layer "F.Cu") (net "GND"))
 (segment (start 167.69 25.96) (end 165.5 25.96) (width 0.2) (layer "F.Cu") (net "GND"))
 (segment (start 170 45.5) (end 167 45.5) (width 0.2) (layer "F.Cu") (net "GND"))
 (segment (start 166 46.5) (end 167 45.5) (width 0.2) (layer "F.Cu") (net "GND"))
 (segment (start 166.5 76.5) (end 167 77) (width 0.2) (layer "F.Cu") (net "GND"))
 (segment (start 166.5 65) (end 166.5 76.5) (width 0.2) (layer "F.Cu") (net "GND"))
 (segment (start 202.62 42.92) (end 203.455 42.92) (width 0.2) (layer "F.Cu") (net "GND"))
 (segment (start 170.73 65) (end 166.5 65) (width 0.2) (layer "F.Cu") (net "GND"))
 (segment (start 167 45.5) (end 166.5 45.5) (width 0.2) (layer "F.Cu") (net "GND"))
 (segment (start 171.27 27) (end 171.27 28.92) (width 0.2) (layer "F.Cu") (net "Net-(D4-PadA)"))
 (segment (start 171.27 28.92) (end 167.69 32.5) (width 0.2) (layer "F.Cu") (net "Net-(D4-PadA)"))
 (segment (start 187.38 40.38) (end 186.545 40.38) (width 0.2) (layer "F.Cu") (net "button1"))
 (segment (start 157.54 23.42) (end 186.42 23.42) (width 0.2) (layer "F.Cu") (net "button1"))
 (segment (start 186.42 23.42) (end 187.38 24.38) (width 0.2) (layer "F.Cu") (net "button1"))
 (segment (start 187.38 40.38) (end 187.38 24.38) (width 0.2) (layer "F.Cu") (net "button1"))
 (segment (start 187.38 42.92) (end 186.545 42.92) (width 0.2) (layer "F.Cu") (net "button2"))
 (segment (start 187.3 43) (end 187.38 42.92) (width 0.2) (layer "B.Cu") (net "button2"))
 (segment (start 157.5 43) (end 187.3 43) (width 0.2) (layer "B.Cu") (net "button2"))
 (segment (start 187.38 45.46) (end 186.545 45.46) (width 0.2) (layer "F.Cu") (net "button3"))
 (segment (start 157.54 62.92) (end 169.92 62.92) (width 0.2) (layer "B.Cu") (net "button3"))
 (segment (start 169.92 62.92) (end 187.38 45.46) (width 0.2) (layer "B.Cu") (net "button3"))
 (segment (start 173.27 66.19) (end 173.27 65) (width 0.2) (layer "F.Cu") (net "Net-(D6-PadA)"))
 (segment (start 169.46 70) (end 173.27 66.19) (width 0.2) (layer "F.Cu") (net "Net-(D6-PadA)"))
 (segment (start 186.30237 48) (end 172.77 34.46763) (width 0.2) (layer "F.Cu") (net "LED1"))
 (segment (start 172.77 34.46763) (end 172.77 32.5) (width 0.2) (layer "F.Cu") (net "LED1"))
 (segment (start 187.38 48) (end 186.30237 48) (width 0.2) (layer "F.Cu") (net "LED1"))
 (segment (start 187.38 48) (end 186.545 48) (width 0.2) (layer "F.Cu") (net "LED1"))
 (segment (start 186.30237 50.54) (end 187.38 50.54) (width 0.2) (layer "F.Cu") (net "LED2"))
 (segment (start 187.38 50.54) (end 186.545 50.54) (width 0.2) (layer "F.Cu") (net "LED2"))
 (segment (start 174.54 62.30237) (end 186.30237 50.54) (width 0.2) (layer "F.Cu") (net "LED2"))
 (segment (start 174.54 70) (end 174.54 62.30237) (width 0.2) (layer "F.Cu") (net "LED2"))
 (segment (start 179.5 51) (end 182.24692 53.74692) (width 0.2) (layer "F.Cu") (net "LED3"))
 (segment (start 174.04 51) (end 179.5 51) (width 0.2) (layer "F.Cu") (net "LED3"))
 (segment (start 187.38 53.08) (end 186.545 53.08) (width 0.2) (layer "F.Cu") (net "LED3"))
 (via (at 186.3855 53.08) (size 0.6) (drill 0.3) (layers "F.Cu" "B.Cu") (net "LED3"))
 (via (at 182.24692 53.74692) (size 0.6) (drill 0.3) (layers "F.Cu" "B.Cu") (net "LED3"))
 (segment (start 185.71858 53.74692) (end 186.3855 53.08) (width 0.2) (layer "B.Cu") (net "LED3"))
 (segment (start 182.24692 53.74692) (end 185.71858 53.74692) (width 0.2) (layer "B.Cu") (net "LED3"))
 (segment (start 202.62 40.38) (end 203.455 40.38) (width 0.2) (layer "F.Cu") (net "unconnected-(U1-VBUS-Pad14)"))
 (segment (start 187.38 55.62) (end 186.545 55.62) (width 0.2) (layer "F.Cu") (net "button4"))
 (segment (start 157.54 82.5) (end 160.5 82.5) (width 0.2) (layer "B.Cu") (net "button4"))
 (segment (start 160.5 82.5) (end 187.38 55.62) (width 0.2) (layer "B.Cu") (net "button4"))
 (segment (start 168.96 51) (end 168.96 49.08) (width 0.2) (layer "F.Cu") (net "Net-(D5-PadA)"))
 (segment (start 168.96 49.08) (end 172.54 45.5) (width 0.2) (layer "F.Cu") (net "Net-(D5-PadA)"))
 (segment (start 171.04 84.88) (end 167.42 88.5) (width 0.2) (layer "F.Cu") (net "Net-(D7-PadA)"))
 (segment (start 171.04 81.5) (end 171.04 84.88) (width 0.2) (layer "F.Cu") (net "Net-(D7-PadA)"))
 (segment (start 202.62 58.38) (end 202.62 55.62) (width 0.2) (layer "B.Cu") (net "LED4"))
 (segment (start 172.5 88.5) (end 202.62 58.38) (width 0.2) (layer "B.Cu") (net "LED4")))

